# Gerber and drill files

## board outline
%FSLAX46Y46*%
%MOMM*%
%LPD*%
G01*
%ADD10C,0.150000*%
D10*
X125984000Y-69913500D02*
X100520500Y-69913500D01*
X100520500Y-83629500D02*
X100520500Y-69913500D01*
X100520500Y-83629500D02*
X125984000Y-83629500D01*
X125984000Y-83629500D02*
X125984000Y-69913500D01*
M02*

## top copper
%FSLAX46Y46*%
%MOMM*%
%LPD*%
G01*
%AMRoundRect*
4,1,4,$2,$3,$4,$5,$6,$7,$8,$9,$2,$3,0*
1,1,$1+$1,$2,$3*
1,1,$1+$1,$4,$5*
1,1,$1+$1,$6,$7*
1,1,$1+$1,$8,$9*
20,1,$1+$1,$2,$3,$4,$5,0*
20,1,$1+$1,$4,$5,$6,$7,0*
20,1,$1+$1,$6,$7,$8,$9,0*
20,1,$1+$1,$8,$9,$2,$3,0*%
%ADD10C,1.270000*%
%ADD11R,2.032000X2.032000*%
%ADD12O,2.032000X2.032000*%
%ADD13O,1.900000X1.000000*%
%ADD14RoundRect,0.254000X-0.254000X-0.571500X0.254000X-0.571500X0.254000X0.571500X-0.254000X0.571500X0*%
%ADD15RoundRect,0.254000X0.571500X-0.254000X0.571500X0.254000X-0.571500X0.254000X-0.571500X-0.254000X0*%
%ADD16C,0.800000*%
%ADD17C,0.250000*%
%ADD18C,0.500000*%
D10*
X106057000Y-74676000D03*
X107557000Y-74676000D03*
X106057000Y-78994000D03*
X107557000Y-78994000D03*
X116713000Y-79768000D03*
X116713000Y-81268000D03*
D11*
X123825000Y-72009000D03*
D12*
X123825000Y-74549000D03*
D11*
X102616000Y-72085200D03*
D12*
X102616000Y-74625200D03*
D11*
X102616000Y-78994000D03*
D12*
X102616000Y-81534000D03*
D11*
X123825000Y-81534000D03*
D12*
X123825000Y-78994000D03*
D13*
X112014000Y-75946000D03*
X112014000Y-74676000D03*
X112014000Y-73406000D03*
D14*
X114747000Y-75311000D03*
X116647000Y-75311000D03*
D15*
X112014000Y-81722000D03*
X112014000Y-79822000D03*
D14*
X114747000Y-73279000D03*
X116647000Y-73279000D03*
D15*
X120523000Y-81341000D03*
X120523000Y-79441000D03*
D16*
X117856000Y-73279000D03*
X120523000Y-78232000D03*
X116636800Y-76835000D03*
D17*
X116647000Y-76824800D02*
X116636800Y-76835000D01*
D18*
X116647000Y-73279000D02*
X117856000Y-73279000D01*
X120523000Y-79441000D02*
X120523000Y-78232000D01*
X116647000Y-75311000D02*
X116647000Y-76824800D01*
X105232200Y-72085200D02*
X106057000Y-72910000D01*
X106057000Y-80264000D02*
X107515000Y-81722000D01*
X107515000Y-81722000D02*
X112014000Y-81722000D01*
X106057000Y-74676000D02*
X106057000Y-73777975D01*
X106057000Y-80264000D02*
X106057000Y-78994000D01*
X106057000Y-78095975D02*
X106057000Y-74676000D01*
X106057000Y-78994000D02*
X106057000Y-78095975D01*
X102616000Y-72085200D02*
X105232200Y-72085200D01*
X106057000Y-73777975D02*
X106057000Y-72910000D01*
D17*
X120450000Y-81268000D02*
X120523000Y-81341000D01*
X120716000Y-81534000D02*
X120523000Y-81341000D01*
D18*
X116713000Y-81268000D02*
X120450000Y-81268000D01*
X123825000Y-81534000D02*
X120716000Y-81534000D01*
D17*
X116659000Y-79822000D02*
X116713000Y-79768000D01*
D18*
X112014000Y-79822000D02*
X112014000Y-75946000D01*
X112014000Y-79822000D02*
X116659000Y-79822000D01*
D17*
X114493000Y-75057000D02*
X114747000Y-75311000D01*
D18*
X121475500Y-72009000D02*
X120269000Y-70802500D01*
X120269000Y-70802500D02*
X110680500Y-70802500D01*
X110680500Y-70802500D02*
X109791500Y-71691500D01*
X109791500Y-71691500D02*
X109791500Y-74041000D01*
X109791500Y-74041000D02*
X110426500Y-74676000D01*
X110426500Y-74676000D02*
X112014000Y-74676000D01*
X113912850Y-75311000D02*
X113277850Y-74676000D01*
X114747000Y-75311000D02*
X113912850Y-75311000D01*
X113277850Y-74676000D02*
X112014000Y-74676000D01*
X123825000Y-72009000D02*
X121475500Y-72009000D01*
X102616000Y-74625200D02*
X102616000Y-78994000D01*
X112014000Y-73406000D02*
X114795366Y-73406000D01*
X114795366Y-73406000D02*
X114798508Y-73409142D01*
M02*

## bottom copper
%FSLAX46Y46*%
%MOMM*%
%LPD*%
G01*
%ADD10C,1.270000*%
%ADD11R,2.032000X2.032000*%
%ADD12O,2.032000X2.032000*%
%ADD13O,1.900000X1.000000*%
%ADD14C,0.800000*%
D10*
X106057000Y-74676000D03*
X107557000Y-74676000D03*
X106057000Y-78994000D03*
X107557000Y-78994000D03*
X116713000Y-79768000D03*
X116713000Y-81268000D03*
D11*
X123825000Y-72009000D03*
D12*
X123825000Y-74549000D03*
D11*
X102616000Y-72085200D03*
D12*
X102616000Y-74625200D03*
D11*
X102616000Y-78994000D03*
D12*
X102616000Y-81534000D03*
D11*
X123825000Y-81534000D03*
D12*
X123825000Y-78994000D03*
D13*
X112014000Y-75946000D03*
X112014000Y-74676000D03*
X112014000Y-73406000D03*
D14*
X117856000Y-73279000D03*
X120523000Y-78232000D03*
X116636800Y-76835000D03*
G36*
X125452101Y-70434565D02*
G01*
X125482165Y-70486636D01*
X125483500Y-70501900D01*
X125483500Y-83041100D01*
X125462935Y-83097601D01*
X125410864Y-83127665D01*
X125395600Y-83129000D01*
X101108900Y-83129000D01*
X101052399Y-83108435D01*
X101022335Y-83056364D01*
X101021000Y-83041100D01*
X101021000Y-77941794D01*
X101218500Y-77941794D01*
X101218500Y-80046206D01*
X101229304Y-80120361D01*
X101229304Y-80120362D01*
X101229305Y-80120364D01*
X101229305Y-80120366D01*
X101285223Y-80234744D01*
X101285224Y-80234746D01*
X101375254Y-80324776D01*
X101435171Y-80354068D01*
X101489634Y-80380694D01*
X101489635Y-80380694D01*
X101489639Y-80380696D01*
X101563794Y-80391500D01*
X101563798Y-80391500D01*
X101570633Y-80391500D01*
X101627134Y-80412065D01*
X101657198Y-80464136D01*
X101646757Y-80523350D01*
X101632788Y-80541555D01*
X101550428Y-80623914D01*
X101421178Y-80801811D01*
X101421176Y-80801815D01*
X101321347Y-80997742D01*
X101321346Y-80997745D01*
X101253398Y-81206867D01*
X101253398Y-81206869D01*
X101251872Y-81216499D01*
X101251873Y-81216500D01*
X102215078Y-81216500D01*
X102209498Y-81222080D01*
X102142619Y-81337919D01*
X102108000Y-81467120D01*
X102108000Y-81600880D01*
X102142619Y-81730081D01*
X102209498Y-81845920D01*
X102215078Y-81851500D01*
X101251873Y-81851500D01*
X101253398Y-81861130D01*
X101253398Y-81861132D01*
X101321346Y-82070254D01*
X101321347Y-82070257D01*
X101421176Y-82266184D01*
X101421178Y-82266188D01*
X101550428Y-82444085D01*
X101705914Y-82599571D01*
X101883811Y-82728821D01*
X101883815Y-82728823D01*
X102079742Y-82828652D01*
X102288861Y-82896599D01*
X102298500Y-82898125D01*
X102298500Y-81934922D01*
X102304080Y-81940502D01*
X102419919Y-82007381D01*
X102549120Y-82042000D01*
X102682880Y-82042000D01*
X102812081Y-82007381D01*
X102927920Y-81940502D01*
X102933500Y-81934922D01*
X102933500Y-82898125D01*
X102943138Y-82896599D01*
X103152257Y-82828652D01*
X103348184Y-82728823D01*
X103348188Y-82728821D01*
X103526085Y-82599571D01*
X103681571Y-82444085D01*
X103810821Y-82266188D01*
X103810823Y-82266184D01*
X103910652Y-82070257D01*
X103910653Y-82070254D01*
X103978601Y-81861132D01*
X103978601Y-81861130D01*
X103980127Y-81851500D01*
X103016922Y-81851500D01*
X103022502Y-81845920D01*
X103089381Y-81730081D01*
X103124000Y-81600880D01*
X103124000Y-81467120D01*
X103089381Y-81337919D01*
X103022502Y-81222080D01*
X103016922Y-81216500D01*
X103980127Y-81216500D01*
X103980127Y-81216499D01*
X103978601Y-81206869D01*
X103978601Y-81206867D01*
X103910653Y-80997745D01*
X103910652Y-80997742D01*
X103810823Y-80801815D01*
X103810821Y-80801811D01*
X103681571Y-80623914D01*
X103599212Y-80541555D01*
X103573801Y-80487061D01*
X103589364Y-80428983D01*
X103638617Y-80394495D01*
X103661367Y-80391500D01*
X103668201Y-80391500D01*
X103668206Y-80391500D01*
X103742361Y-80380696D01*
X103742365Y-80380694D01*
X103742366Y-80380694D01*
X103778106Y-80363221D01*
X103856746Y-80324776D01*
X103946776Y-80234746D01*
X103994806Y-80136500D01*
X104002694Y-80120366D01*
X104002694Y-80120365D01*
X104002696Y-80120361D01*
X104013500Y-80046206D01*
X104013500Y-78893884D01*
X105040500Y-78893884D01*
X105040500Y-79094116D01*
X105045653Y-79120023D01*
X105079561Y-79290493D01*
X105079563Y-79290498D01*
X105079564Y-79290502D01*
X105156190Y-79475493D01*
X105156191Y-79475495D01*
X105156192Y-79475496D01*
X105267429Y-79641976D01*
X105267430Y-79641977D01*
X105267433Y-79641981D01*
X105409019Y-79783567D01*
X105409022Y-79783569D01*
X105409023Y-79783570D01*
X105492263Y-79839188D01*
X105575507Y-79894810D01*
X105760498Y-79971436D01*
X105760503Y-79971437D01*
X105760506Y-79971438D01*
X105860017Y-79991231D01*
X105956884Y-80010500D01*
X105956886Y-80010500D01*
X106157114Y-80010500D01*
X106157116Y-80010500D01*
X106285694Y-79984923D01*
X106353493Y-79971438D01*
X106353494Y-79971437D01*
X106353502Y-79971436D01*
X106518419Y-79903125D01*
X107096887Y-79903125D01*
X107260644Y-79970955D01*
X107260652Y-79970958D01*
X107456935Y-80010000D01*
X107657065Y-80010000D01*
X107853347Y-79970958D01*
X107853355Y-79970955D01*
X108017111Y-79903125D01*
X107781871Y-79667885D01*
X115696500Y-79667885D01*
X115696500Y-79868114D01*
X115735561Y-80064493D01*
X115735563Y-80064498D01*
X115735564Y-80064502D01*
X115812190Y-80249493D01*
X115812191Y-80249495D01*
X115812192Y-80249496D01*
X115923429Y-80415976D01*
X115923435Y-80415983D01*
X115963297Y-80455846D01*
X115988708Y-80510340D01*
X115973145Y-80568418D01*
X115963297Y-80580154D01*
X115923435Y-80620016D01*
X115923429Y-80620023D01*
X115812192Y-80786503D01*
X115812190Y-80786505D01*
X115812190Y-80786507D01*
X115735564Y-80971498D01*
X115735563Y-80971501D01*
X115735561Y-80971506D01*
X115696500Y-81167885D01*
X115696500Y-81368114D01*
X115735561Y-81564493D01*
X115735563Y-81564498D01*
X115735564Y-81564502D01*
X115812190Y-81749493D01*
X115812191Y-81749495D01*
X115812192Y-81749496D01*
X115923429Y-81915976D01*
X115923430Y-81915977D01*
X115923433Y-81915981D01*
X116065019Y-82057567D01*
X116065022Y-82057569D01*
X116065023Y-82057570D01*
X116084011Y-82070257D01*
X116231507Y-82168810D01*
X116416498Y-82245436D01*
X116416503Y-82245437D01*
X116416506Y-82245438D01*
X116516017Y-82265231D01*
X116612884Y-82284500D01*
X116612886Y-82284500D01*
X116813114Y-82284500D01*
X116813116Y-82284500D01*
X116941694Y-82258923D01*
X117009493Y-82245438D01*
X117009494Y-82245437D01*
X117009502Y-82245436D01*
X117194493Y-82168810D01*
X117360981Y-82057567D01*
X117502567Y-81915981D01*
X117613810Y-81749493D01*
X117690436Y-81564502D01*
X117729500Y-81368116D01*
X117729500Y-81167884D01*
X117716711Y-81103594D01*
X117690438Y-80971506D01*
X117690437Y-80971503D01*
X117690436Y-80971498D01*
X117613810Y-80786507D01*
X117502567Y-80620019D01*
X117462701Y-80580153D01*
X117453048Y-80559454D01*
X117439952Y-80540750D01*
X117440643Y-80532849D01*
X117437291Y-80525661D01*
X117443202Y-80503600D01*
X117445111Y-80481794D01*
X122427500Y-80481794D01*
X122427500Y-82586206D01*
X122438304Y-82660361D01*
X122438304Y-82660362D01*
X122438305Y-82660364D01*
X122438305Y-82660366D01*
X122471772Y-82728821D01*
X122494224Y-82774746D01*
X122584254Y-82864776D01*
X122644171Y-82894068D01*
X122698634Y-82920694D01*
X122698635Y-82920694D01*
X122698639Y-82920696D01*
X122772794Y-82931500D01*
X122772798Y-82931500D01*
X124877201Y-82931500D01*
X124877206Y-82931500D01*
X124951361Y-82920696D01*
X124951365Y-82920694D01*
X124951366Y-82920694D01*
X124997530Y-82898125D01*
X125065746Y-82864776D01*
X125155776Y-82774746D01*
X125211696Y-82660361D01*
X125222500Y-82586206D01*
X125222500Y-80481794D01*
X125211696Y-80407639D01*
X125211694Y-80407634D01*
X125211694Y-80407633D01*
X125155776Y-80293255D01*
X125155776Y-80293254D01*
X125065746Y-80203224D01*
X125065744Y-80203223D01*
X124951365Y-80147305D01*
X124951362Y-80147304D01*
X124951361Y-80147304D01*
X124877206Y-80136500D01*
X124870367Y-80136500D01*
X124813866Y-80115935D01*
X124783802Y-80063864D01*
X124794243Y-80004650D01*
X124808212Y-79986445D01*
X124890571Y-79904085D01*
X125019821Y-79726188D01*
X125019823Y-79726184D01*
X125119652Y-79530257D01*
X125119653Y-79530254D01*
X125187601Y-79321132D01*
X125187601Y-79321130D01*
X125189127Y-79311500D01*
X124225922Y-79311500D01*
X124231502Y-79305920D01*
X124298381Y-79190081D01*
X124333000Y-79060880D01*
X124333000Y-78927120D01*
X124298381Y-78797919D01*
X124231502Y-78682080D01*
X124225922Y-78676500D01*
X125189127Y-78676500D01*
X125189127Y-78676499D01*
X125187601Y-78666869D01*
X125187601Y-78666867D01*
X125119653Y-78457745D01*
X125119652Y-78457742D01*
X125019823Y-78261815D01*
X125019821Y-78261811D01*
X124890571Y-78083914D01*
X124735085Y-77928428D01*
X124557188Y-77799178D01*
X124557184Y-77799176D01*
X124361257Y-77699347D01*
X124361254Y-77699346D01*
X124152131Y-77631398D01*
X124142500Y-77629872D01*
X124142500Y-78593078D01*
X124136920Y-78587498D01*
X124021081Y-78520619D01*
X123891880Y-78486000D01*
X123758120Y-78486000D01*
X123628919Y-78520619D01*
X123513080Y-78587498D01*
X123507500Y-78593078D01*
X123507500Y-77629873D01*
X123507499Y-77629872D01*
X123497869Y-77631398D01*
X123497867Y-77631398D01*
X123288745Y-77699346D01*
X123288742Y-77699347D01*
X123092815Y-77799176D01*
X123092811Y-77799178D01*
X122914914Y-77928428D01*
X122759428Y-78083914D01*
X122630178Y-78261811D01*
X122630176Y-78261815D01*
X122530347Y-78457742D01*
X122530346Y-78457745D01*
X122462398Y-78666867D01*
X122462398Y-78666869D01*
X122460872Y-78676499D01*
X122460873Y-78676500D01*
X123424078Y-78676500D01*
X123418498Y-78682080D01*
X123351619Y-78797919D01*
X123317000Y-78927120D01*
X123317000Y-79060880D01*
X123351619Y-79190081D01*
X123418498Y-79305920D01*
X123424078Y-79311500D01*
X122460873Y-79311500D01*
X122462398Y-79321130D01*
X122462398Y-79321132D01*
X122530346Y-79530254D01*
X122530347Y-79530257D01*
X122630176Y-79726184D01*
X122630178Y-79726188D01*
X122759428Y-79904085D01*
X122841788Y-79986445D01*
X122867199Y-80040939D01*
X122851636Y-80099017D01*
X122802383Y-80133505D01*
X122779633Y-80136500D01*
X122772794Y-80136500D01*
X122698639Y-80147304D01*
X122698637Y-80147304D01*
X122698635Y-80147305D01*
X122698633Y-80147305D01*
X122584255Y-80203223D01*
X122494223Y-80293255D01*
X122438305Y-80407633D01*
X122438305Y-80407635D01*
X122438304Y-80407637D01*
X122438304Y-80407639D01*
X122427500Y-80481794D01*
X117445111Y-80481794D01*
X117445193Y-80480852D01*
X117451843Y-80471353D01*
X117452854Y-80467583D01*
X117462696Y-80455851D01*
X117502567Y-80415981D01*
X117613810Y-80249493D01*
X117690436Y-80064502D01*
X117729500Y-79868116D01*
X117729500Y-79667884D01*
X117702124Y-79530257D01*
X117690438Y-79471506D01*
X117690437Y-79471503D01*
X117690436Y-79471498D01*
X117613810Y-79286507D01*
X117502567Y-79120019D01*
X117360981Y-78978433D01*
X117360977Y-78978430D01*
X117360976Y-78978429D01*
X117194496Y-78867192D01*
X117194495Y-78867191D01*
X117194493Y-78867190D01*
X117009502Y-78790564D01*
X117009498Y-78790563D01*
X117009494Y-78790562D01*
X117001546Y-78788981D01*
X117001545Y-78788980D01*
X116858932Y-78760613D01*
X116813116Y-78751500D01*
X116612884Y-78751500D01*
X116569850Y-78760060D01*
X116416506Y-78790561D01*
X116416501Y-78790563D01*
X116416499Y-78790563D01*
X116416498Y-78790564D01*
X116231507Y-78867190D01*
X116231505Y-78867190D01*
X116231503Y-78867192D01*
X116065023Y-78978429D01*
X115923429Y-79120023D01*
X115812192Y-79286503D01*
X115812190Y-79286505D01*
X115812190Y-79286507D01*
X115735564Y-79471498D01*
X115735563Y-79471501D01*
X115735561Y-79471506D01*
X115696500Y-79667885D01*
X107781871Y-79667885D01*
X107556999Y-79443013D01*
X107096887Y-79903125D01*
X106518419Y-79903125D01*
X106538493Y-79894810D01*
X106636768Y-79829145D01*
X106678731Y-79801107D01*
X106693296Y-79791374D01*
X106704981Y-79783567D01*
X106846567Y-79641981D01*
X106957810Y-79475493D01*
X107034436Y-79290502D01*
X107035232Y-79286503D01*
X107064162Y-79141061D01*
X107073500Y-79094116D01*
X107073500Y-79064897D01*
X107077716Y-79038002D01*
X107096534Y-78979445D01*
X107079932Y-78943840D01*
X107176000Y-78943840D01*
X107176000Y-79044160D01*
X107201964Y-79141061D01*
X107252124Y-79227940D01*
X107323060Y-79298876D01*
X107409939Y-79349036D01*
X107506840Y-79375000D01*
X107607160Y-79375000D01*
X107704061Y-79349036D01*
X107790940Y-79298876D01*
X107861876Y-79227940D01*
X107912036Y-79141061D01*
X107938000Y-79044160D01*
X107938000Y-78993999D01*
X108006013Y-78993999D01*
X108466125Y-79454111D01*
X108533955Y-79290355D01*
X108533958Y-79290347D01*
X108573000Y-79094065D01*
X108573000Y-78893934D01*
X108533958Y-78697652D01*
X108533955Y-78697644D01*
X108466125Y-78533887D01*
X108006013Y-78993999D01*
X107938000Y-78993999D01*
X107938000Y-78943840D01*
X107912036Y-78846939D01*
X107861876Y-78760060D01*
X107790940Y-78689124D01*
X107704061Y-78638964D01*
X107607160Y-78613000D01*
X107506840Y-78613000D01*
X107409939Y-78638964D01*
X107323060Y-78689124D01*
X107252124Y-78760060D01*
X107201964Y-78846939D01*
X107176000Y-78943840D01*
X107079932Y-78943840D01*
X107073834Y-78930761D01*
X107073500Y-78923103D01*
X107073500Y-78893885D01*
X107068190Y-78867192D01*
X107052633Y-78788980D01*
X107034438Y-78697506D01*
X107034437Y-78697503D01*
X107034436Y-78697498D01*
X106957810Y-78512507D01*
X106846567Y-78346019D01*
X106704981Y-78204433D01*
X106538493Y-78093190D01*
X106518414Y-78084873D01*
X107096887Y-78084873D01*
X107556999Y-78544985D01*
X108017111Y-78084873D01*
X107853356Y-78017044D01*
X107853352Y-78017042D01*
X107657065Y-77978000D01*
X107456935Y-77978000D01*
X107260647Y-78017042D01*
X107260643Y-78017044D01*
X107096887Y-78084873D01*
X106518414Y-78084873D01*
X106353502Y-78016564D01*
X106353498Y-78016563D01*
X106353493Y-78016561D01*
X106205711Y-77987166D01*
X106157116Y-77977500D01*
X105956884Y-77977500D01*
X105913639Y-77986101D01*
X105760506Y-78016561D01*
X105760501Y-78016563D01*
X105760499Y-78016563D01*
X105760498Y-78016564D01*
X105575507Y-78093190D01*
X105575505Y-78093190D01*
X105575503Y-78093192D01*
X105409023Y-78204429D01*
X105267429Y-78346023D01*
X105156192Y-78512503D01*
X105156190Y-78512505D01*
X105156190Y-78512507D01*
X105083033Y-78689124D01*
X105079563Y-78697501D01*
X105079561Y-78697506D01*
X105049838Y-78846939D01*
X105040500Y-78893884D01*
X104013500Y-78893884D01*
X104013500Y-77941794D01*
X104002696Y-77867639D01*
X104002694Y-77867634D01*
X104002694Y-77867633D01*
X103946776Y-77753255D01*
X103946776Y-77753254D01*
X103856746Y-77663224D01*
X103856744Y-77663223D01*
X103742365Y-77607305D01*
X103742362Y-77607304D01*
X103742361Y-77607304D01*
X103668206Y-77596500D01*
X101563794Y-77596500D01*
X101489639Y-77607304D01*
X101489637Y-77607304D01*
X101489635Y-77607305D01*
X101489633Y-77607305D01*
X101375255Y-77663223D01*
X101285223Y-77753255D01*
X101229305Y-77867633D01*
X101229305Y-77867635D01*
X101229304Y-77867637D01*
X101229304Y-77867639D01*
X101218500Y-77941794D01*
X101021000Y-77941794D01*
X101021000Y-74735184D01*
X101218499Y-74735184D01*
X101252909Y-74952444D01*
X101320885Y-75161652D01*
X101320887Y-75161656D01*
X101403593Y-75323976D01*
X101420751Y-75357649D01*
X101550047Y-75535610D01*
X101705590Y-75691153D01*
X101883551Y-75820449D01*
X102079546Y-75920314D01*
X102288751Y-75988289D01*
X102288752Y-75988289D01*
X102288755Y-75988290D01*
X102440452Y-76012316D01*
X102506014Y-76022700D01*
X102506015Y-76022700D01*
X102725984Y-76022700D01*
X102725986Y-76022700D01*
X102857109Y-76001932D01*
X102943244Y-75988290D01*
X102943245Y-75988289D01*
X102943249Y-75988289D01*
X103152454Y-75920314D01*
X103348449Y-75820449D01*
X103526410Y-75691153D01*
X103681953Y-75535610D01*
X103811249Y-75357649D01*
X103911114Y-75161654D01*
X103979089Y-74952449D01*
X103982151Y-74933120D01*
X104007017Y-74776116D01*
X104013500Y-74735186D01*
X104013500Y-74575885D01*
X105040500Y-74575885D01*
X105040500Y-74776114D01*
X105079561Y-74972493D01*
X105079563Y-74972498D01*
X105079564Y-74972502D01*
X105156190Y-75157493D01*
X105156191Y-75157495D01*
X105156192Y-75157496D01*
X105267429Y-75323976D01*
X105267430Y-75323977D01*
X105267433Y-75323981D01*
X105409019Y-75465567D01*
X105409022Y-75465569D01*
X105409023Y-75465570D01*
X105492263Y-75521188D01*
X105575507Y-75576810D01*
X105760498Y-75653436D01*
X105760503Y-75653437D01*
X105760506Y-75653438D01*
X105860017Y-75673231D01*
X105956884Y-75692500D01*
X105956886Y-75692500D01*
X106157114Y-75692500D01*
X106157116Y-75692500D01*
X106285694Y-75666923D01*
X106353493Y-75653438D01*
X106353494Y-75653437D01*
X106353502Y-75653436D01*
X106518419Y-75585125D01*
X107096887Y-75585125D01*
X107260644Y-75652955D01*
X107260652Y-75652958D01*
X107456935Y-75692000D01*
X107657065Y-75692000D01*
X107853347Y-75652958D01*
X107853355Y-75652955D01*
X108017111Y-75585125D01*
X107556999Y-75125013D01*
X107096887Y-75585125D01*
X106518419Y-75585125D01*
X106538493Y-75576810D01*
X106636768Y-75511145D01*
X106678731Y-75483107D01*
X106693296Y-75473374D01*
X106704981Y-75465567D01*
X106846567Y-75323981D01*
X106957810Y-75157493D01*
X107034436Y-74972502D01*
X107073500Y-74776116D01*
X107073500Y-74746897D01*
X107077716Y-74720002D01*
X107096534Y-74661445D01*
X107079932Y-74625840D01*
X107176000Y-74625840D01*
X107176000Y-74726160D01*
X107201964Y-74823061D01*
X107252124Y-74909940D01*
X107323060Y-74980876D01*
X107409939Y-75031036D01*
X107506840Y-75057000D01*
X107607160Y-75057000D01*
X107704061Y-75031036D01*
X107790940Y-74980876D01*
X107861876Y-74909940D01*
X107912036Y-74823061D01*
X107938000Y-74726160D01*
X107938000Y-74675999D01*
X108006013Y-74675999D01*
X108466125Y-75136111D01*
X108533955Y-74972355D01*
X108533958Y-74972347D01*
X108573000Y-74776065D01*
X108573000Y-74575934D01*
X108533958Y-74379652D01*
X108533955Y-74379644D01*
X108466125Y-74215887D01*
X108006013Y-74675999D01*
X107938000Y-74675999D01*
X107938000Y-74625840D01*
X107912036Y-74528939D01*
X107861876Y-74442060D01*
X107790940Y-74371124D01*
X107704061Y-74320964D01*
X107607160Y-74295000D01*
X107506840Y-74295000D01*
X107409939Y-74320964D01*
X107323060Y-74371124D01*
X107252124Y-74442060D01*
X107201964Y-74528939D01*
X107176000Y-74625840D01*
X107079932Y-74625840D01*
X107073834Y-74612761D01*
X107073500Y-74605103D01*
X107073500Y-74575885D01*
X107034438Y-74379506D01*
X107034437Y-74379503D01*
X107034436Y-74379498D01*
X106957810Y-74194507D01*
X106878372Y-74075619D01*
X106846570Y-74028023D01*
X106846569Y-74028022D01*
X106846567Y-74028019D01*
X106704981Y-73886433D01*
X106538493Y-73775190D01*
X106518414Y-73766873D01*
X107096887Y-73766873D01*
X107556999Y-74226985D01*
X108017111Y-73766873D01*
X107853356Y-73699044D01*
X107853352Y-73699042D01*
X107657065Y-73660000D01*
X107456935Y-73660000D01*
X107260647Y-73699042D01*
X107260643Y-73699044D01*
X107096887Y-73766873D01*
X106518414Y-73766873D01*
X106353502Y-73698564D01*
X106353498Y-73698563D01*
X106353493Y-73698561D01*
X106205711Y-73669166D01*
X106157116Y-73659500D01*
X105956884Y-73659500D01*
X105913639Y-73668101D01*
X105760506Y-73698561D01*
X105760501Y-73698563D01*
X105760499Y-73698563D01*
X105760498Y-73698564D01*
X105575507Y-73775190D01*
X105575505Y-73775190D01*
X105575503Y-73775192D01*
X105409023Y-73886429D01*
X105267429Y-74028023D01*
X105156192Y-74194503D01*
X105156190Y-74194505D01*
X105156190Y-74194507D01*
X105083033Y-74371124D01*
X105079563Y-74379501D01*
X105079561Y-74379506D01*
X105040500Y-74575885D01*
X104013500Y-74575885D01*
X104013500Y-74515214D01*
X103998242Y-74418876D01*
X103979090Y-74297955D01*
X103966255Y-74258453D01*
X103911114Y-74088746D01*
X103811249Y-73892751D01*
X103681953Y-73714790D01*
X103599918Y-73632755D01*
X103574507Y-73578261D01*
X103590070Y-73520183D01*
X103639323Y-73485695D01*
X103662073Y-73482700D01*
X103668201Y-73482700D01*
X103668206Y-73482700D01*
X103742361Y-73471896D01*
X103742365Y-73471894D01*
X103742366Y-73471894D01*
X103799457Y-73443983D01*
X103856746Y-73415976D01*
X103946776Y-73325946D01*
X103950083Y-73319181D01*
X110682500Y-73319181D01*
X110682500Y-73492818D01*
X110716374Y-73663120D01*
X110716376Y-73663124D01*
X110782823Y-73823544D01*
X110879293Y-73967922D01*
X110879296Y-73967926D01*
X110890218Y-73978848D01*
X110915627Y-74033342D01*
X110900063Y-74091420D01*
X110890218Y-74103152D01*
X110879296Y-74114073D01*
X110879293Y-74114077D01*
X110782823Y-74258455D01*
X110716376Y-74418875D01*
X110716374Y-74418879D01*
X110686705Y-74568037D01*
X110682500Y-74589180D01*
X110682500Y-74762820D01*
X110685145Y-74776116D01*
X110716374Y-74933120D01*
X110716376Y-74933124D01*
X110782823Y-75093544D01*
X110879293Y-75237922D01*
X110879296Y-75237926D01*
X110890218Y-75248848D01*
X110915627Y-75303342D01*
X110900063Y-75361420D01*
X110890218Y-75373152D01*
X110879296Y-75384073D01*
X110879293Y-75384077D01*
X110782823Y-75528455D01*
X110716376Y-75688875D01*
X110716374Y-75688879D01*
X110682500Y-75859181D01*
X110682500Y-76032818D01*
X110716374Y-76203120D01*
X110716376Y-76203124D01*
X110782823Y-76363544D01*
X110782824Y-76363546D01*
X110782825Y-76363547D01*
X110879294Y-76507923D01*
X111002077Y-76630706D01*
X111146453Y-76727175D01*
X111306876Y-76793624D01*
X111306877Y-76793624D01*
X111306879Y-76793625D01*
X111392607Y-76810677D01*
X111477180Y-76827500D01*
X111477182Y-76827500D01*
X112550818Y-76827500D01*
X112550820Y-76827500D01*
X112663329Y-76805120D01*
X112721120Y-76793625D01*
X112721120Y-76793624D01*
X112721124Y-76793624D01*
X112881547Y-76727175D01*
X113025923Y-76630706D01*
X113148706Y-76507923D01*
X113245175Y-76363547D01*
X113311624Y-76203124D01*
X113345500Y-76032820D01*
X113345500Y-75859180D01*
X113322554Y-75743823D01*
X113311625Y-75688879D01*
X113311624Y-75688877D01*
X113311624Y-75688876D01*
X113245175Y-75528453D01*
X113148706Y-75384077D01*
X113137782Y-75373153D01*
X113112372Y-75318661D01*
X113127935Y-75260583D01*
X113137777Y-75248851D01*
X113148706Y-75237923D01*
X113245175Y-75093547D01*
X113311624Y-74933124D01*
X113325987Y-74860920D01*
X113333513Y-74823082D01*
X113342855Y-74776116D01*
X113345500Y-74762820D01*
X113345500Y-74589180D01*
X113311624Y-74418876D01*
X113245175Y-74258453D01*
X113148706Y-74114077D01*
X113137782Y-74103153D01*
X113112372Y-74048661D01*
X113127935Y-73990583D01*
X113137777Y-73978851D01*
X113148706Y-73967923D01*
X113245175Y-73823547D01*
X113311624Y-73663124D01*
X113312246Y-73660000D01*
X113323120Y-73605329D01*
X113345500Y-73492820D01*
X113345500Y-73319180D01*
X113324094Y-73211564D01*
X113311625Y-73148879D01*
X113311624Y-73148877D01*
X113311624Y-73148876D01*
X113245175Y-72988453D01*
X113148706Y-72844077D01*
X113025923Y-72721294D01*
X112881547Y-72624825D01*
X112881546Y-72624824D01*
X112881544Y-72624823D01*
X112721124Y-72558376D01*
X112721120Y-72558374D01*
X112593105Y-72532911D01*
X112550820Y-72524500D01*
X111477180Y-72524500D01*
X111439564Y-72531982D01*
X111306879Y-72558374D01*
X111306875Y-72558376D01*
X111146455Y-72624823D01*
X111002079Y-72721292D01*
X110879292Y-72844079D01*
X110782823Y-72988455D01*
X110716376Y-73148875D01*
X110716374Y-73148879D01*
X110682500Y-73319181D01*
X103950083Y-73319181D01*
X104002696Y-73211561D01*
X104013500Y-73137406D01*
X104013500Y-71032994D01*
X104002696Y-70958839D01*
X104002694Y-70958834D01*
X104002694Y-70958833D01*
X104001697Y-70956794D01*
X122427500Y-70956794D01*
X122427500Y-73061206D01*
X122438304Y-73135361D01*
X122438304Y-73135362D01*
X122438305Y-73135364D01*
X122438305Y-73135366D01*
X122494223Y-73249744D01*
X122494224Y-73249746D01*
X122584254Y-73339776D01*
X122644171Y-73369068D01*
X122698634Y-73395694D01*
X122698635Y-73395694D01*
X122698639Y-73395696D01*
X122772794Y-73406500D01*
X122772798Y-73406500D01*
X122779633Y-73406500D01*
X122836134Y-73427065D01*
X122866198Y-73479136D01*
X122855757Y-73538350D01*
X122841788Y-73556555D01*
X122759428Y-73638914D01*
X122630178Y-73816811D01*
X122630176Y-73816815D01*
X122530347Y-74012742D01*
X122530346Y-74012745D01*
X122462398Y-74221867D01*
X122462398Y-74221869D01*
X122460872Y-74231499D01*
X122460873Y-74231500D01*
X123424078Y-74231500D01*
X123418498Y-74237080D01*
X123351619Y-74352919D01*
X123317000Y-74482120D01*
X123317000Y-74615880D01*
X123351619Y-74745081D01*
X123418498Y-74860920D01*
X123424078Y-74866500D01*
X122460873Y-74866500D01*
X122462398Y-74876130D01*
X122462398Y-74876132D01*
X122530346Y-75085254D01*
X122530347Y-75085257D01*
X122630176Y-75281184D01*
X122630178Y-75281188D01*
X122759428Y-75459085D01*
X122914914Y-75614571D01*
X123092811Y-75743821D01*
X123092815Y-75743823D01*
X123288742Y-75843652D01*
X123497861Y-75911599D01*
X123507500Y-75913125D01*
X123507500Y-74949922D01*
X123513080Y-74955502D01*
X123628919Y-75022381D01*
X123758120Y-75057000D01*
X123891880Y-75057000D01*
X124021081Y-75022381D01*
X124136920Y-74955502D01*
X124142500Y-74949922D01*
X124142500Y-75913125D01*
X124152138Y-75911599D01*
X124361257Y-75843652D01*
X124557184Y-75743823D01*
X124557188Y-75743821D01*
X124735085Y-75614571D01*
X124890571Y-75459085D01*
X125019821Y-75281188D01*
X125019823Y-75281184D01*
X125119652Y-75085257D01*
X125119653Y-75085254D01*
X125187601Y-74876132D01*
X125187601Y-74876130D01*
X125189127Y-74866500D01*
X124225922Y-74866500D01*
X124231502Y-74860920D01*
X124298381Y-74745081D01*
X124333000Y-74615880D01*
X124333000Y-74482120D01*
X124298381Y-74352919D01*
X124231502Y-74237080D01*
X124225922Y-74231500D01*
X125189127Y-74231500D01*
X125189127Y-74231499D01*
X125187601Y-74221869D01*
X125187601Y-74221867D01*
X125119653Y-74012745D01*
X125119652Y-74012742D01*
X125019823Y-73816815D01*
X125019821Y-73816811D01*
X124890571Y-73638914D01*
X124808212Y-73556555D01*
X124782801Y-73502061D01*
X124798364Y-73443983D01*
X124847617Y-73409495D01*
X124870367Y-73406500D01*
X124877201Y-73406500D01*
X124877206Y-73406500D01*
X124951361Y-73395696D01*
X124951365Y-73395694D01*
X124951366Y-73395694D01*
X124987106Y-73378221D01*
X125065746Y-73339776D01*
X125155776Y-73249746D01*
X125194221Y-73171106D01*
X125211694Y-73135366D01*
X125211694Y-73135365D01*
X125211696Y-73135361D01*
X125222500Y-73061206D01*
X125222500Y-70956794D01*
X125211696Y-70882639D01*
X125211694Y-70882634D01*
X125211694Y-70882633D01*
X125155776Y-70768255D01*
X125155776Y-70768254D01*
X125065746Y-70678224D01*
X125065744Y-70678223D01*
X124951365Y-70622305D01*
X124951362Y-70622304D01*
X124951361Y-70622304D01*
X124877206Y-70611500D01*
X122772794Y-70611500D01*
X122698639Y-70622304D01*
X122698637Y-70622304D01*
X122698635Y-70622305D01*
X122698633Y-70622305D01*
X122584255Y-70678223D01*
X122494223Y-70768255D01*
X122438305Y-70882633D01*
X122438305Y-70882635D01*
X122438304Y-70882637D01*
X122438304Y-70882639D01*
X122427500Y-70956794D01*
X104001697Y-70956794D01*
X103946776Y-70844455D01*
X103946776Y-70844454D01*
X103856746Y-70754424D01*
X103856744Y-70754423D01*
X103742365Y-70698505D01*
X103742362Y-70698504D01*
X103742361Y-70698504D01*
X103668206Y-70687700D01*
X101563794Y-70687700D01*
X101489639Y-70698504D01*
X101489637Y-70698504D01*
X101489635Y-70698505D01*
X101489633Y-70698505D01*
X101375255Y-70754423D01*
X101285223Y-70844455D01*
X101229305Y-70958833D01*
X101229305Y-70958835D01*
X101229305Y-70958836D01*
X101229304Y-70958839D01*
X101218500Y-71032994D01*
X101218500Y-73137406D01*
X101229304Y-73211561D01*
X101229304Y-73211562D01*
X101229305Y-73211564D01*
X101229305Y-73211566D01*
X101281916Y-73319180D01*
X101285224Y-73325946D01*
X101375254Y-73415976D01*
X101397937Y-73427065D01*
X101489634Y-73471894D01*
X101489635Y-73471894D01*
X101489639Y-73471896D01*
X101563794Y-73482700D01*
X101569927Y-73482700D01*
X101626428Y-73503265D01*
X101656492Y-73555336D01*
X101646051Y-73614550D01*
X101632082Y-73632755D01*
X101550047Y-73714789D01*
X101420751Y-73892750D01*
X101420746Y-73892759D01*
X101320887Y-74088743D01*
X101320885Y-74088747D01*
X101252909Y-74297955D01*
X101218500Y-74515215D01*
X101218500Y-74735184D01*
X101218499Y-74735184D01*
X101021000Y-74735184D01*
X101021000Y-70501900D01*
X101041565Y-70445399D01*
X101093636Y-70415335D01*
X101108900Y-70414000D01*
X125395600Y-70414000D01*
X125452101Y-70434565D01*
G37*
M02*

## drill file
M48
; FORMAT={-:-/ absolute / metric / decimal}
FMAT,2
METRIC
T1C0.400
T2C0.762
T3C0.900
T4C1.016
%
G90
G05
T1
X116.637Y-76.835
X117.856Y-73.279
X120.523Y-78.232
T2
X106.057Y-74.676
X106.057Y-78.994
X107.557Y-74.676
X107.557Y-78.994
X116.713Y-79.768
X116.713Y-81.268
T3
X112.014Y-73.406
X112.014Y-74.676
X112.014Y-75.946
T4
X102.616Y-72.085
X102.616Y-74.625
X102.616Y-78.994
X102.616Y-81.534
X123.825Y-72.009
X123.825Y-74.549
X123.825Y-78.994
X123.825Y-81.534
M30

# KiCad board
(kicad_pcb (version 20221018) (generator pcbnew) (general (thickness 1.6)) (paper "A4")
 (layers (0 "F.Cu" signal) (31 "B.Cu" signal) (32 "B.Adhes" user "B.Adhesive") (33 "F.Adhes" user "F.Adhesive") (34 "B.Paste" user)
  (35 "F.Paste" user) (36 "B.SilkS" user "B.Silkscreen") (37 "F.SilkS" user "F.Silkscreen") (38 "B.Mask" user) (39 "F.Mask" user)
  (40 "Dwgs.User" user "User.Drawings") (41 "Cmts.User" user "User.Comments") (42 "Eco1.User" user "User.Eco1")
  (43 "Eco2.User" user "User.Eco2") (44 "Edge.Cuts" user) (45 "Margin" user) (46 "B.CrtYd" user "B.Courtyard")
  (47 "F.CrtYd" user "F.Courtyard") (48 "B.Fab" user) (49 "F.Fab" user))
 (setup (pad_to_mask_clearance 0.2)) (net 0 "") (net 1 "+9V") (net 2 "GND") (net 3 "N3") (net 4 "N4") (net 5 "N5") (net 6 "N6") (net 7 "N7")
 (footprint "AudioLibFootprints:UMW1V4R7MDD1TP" (layer "F.Cu") (at 106.807 74.676)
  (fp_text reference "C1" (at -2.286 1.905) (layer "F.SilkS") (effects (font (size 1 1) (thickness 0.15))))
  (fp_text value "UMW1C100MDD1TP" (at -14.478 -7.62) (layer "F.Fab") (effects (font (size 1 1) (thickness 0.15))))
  (pad "1" thru_hole circle (at -0.75 0) (size 1.27 1.27) (drill 0.762) (layers "*.Cu" "*.Mask") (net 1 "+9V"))
  (pad "2" thru_hole circle (at 0.75 0) (size 1.27 1.27) (drill 0.762) (layers "*.Cu" "*.Mask") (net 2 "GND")))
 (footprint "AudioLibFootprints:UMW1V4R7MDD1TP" (layer "F.Cu") (at 106.807 78.994)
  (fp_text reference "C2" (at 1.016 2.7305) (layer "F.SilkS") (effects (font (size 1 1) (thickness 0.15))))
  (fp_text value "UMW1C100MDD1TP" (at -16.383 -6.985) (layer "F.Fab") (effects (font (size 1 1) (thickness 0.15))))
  (pad "1" thru_hole circle (at -0.75 0) (size 1.27 1.27) (drill 0.762) (layers "*.Cu" "*.Mask") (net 1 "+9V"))
  (pad "2" thru_hole circle (at 0.75 0) (size 1.27 1.27) (drill 0.762) (layers "*.Cu" "*.Mask") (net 2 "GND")))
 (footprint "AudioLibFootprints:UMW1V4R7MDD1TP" (layer "F.Cu") (at 116.713 80.518 -90)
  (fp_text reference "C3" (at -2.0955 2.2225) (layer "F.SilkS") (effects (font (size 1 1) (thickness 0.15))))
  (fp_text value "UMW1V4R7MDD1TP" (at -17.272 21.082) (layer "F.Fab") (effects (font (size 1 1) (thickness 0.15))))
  (pad "1" thru_hole circle (at -0.75 0 270) (size 1.27 1.27) (drill 0.762) (layers "*.Cu" "*.Mask") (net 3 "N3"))
  (pad "2" thru_hole circle (at 0.75 0 270) (size 1.27 1.27) (drill 0.762) (layers "*.Cu" "*.Mask") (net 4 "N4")))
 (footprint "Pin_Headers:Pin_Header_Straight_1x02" (layer "F.Cu") (at 123.825 72.009)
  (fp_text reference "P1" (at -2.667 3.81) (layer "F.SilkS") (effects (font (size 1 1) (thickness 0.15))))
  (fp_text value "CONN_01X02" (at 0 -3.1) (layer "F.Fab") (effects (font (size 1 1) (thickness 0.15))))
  (pad "1" thru_hole rect (at 0 0) (size 2.032 2.032) (drill 1.016) (layers "*.Cu" "*.Mask" "F.SilkS") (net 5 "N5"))
  (pad "2" thru_hole oval (at 0 2.54) (size 2.032 2.032) (drill 1.016) (layers "*.Cu" "*.Mask" "F.SilkS") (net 2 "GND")))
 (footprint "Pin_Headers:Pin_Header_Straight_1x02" (layer "F.Cu") (at 102.616 72.0852)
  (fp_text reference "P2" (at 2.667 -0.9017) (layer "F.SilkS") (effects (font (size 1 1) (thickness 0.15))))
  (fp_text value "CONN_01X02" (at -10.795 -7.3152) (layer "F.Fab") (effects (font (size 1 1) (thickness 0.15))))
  (pad "1" thru_hole rect (at 0 0) (size 2.032 2.032) (drill 1.016) (layers "*.Cu" "*.Mask" "F.SilkS") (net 1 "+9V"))
  (pad "2" thru_hole oval (at 0 2.54) (size 2.032 2.032) (drill 1.016) (layers "*.Cu" "*.Mask" "F.SilkS") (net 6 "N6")))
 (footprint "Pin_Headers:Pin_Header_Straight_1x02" (layer "F.Cu") (at 102.616 78.994)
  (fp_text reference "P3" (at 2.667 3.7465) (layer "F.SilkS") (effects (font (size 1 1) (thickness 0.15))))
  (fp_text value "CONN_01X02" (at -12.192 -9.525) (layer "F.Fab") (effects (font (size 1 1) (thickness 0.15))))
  (pad "1" thru_hole rect (at 0 0) (size 2.032 2.032) (drill 1.016) (layers "*.Cu" "*.Mask" "F.SilkS") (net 6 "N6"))
  (pad "2" thru_hole oval (at 0 2.54) (size 2.032 2.032) (drill 1.016) (layers "*.Cu" "*.Mask" "F.SilkS") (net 2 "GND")))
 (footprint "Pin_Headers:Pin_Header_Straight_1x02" (layer "F.Cu") (at 123.825 81.534 180)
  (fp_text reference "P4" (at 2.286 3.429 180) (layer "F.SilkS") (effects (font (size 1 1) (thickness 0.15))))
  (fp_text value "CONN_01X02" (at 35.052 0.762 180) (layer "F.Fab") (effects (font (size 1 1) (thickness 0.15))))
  (pad "1" thru_hole rect (at 0 0 180) (size 2.032 2.032) (drill 1.016) (layers "*.Cu" "*.Mask" "F.SilkS") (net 4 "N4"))
  (pad "2" thru_hole oval (at 0 2.54 180) (size 2.032 2.032) (drill 1.016) (layers "*.Cu" "*.Mask" "F.SilkS") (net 2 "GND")))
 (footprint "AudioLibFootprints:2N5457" (layer "F.Cu") (at 112.014 74.676)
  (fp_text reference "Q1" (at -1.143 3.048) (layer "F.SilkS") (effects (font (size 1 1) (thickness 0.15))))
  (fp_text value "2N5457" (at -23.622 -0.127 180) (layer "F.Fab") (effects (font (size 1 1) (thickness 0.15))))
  (pad "1" thru_hole oval (at 0 1.27) (size 1.9 1) (drill 0.9) (layers "*.Cu" "*.Mask") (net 3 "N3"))
  (pad "2" thru_hole oval (at 0 0) (size 1.9 1) (drill 0.9) (layers "*.Cu" "*.Mask") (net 5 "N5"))
  (pad "3" thru_hole oval (at 0 -1.27) (size 1.9 1) (drill 0.9) (layers "*.Cu" "*.Mask") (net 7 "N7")))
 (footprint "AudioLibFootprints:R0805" (layer "F.Cu") (at 115.697 75.311)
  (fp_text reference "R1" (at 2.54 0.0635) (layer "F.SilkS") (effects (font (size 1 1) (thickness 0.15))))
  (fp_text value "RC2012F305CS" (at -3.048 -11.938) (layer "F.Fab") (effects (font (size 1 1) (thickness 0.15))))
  (pad "1" smd roundrect (at -0.95 0) (size 1.016 1.651) (layers "F.Cu" "F.Paste" "F.Mask") (roundrect_rratio 0.25) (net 5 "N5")
   (solder_mask_margin 0.102))
  (pad "2" smd roundrect (at 0.95 0) (size 1.016 1.651) (layers "F.Cu" "F.Paste" "F.Mask") (roundrect_rratio 0.25) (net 2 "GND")
   (solder_mask_margin 0.102)))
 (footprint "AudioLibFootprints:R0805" (layer "F.Cu") (at 112.014 80.772 90)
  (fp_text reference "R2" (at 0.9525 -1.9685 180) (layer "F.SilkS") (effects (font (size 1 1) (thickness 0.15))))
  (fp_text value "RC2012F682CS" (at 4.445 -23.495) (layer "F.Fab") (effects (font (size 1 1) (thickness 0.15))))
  (pad "1" smd roundrect (at -0.95 0 90) (size 1.016 1.651) (layers "F.Cu" "F.Paste" "F.Mask") (roundrect_rratio 0.25) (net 1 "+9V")
   (solder_mask_margin 0.102))
  (pad "2" smd roundrect (at 0.95 0 90) (size 1.016 1.651) (layers "F.Cu" "F.Paste" "F.Mask") (roundrect_rratio 0.25) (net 3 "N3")
   (solder_mask_margin 0.102)))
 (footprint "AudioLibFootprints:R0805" (layer "F.Cu") (at 115.697 73.279)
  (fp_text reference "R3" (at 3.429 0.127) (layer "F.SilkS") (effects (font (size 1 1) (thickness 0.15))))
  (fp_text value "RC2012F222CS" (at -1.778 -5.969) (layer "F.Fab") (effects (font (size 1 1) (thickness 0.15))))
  (pad "1" smd roundrect (at -0.95 0) (size 1.016 1.651) (layers "F.Cu" "F.Paste" "F.Mask") (roundrect_rratio 0.25) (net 7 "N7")
   (solder_mask_margin 0.102))
  (pad "2" smd roundrect (at 0.95 0) (size 1.016 1.651) (layers "F.Cu" "F.Paste" "F.Mask") (roundrect_rratio 0.25) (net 2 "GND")
   (solder_mask_margin 0.102)))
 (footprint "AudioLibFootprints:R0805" (layer "F.Cu") (at 120.523 80.391 90)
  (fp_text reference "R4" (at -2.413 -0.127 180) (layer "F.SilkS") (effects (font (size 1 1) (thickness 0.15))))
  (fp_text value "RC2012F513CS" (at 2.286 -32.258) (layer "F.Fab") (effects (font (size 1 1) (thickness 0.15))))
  (pad "1" smd roundrect (at -0.95 0 90) (size 1.016 1.651) (layers "F.Cu" "F.Paste" "F.Mask") (roundrect_rratio 0.25) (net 4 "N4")
   (solder_mask_margin 0.102))
  (pad "2" smd roundrect (at 0.95 0 90) (size 1.016 1.651) (layers "F.Cu" "F.Paste" "F.Mask") (roundrect_rratio 0.25) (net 2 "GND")
   (solder_mask_margin 0.102)))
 (gr_line (start 125.984 69.9135) (end 100.5205 69.9135) (stroke (width 0.15) (type solid)) (layer "Edge.Cuts"))
 (gr_line (start 100.5205 83.6295) (end 100.5205 69.9135) (stroke (width 0.15) (type solid)) (layer "Edge.Cuts"))
 (gr_line (start 100.5205 83.6295) (end 125.984 83.6295) (stroke (width 0.15) (type solid)) (layer "Edge.Cuts"))
 (gr_line (start 125.984 83.6295) (end 125.984 69.9135) (stroke (width 0.15) (type solid)) (layer "Edge.Cuts"))
 (segment (start 116.647 76.8248) (end 116.6368 76.835) (width 0.25) (layer "F.Cu") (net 2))
 (segment (start 116.647 73.279) (end 117.856 73.279) (width 0.5) (layer "F.Cu") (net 2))
 (segment (start 120.523 79.441) (end 120.523 78.232) (width 0.5) (layer "F.Cu") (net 2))
 (segment (start 116.647 75.311) (end 116.647 76.8248) (width 0.5) (layer "F.Cu") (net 2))
 (via (at 117.856 73.279) (size 0.8) (drill 0.4) (layers "F.Cu" "B.Cu") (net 2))
 (via (at 120.523 78.232) (size 0.8) (drill 0.4) (layers "F.Cu" "B.Cu") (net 2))
 (via (at 116.6368 76.835) (size 0.8) (drill 0.4) (layers "F.Cu" "B.Cu") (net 2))
 (segment (start 105.2322 72.0852) (end 106.057 72.91) (width 0.5) (layer "F.Cu") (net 1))
 (segment (start 106.057 80.264) (end 107.515 81.722) (width 0.5) (layer "F.Cu") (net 1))
 (segment (start 107.515 81.722) (end 112.014 81.722) (width 0.5) (layer "F.Cu") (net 1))
 (segment (start 106.057 74.676) (end 106.057 73.777975) (width 0.5) (layer "F.Cu") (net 1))
 (segment (start 106.057 80.264) (end 106.057 78.994) (width 0.5) (layer "F.Cu") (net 1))
 (segment (start 106.057 78.095975) (end 106.057 74.676) (width 0.5) (layer "F.Cu") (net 1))
 (segment (start 106.057 78.994) (end 106.057 78.095975) (width 0.5) (layer "F.Cu") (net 1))
 (segment (start 102.616 72.0852) (end 105.2322 72.0852) (width 0.5) (layer "F.Cu") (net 1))
 (segment (start 106.057 73.777975) (end 106.057 72.91) (width 0.5) (layer "F.Cu") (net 1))
 (segment (start 120.45 81.268) (end 120.523 81.341) (width 0.25) (layer "F.Cu") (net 4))
 (segment (start 120.716 81.534) (end 120.523 81.341) (width 0.25) (layer "F.Cu") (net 4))
 (segment (start 116.713 81.268) (end 120.45 81.268) (width 0.5) (layer "F.Cu") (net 4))
 (segment (start 123.825 81.534) (end 120.716 81.534) (width 0.5) (layer "F.Cu") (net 4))
 (segment (start 116.659 79.822) (end 116.713 79.768) (width 0.25) (layer "F.Cu") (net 3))
 (segment (start 112.014 79.822) (end 112.014 75.946) (width 0.5) (layer "F.Cu") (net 3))
 (segment (start 112.014 79.822) (end 116.659 79.822) (width 0.5) (layer "F.Cu") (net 3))
 (segment (start 114.493 75.057) (end 114.747 75.311) (width 0.25) (layer "F.Cu") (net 5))
 (segment (start 121.4755 72.009) (end 120.269 70.8025) (width 0.5) (layer "F.Cu") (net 5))
 (segment (start 120.269 70.8025) (end 110.6805 70.8025) (width 0.5) (layer "F.Cu") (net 5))
 (segment (start 110.6805 70.8025) (end 109.7915 71.6915) (width 0.5) (layer "F.Cu") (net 5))
 (segment (start 109.7915 71.6915) (end 109.7915 74.041) (width 0.5) (layer "F.Cu") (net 5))
 (segment (start 109.7915 74.041) (end 110.4265 74.676) (width 0.5) (layer "F.Cu") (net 5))
 (segment (start 110.4265 74.676) (end 112.014 74.676) (width 0.5) (layer "F.Cu") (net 5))
 (segment (start 113.91285 75.311) (end 113.27785 74.676) (width 0.5) (layer "F.Cu") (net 5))
 (segment (start 114.747 75.311) (end 113.91285 75.311) (width 0.5) (layer "F.Cu") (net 5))
 (segment (start 113.27785 74.676) (end 112.014 74.676) (width 0.5) (layer "F.Cu") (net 5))
 (segment (start 123.825 72.009) (end 121.4755 72.009) (width 0.5) (layer "F.Cu") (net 5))
 (segment (start 102.616 74.6252) (end 102.616 78.994) (width 0.5) (layer "F.Cu") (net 6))
 (segment (start 112.014 73.406) (end 114.795366 73.406) (width 0.5) (layer "F.Cu") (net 7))
 (segment (start 114.795366 73.406) (end 114.798508 73.409142) (width 0.5) (layer "F.Cu") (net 7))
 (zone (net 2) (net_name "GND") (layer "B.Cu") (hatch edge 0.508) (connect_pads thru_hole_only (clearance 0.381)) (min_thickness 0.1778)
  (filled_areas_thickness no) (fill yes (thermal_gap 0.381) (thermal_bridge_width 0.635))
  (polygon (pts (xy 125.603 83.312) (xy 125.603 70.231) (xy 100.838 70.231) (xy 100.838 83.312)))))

